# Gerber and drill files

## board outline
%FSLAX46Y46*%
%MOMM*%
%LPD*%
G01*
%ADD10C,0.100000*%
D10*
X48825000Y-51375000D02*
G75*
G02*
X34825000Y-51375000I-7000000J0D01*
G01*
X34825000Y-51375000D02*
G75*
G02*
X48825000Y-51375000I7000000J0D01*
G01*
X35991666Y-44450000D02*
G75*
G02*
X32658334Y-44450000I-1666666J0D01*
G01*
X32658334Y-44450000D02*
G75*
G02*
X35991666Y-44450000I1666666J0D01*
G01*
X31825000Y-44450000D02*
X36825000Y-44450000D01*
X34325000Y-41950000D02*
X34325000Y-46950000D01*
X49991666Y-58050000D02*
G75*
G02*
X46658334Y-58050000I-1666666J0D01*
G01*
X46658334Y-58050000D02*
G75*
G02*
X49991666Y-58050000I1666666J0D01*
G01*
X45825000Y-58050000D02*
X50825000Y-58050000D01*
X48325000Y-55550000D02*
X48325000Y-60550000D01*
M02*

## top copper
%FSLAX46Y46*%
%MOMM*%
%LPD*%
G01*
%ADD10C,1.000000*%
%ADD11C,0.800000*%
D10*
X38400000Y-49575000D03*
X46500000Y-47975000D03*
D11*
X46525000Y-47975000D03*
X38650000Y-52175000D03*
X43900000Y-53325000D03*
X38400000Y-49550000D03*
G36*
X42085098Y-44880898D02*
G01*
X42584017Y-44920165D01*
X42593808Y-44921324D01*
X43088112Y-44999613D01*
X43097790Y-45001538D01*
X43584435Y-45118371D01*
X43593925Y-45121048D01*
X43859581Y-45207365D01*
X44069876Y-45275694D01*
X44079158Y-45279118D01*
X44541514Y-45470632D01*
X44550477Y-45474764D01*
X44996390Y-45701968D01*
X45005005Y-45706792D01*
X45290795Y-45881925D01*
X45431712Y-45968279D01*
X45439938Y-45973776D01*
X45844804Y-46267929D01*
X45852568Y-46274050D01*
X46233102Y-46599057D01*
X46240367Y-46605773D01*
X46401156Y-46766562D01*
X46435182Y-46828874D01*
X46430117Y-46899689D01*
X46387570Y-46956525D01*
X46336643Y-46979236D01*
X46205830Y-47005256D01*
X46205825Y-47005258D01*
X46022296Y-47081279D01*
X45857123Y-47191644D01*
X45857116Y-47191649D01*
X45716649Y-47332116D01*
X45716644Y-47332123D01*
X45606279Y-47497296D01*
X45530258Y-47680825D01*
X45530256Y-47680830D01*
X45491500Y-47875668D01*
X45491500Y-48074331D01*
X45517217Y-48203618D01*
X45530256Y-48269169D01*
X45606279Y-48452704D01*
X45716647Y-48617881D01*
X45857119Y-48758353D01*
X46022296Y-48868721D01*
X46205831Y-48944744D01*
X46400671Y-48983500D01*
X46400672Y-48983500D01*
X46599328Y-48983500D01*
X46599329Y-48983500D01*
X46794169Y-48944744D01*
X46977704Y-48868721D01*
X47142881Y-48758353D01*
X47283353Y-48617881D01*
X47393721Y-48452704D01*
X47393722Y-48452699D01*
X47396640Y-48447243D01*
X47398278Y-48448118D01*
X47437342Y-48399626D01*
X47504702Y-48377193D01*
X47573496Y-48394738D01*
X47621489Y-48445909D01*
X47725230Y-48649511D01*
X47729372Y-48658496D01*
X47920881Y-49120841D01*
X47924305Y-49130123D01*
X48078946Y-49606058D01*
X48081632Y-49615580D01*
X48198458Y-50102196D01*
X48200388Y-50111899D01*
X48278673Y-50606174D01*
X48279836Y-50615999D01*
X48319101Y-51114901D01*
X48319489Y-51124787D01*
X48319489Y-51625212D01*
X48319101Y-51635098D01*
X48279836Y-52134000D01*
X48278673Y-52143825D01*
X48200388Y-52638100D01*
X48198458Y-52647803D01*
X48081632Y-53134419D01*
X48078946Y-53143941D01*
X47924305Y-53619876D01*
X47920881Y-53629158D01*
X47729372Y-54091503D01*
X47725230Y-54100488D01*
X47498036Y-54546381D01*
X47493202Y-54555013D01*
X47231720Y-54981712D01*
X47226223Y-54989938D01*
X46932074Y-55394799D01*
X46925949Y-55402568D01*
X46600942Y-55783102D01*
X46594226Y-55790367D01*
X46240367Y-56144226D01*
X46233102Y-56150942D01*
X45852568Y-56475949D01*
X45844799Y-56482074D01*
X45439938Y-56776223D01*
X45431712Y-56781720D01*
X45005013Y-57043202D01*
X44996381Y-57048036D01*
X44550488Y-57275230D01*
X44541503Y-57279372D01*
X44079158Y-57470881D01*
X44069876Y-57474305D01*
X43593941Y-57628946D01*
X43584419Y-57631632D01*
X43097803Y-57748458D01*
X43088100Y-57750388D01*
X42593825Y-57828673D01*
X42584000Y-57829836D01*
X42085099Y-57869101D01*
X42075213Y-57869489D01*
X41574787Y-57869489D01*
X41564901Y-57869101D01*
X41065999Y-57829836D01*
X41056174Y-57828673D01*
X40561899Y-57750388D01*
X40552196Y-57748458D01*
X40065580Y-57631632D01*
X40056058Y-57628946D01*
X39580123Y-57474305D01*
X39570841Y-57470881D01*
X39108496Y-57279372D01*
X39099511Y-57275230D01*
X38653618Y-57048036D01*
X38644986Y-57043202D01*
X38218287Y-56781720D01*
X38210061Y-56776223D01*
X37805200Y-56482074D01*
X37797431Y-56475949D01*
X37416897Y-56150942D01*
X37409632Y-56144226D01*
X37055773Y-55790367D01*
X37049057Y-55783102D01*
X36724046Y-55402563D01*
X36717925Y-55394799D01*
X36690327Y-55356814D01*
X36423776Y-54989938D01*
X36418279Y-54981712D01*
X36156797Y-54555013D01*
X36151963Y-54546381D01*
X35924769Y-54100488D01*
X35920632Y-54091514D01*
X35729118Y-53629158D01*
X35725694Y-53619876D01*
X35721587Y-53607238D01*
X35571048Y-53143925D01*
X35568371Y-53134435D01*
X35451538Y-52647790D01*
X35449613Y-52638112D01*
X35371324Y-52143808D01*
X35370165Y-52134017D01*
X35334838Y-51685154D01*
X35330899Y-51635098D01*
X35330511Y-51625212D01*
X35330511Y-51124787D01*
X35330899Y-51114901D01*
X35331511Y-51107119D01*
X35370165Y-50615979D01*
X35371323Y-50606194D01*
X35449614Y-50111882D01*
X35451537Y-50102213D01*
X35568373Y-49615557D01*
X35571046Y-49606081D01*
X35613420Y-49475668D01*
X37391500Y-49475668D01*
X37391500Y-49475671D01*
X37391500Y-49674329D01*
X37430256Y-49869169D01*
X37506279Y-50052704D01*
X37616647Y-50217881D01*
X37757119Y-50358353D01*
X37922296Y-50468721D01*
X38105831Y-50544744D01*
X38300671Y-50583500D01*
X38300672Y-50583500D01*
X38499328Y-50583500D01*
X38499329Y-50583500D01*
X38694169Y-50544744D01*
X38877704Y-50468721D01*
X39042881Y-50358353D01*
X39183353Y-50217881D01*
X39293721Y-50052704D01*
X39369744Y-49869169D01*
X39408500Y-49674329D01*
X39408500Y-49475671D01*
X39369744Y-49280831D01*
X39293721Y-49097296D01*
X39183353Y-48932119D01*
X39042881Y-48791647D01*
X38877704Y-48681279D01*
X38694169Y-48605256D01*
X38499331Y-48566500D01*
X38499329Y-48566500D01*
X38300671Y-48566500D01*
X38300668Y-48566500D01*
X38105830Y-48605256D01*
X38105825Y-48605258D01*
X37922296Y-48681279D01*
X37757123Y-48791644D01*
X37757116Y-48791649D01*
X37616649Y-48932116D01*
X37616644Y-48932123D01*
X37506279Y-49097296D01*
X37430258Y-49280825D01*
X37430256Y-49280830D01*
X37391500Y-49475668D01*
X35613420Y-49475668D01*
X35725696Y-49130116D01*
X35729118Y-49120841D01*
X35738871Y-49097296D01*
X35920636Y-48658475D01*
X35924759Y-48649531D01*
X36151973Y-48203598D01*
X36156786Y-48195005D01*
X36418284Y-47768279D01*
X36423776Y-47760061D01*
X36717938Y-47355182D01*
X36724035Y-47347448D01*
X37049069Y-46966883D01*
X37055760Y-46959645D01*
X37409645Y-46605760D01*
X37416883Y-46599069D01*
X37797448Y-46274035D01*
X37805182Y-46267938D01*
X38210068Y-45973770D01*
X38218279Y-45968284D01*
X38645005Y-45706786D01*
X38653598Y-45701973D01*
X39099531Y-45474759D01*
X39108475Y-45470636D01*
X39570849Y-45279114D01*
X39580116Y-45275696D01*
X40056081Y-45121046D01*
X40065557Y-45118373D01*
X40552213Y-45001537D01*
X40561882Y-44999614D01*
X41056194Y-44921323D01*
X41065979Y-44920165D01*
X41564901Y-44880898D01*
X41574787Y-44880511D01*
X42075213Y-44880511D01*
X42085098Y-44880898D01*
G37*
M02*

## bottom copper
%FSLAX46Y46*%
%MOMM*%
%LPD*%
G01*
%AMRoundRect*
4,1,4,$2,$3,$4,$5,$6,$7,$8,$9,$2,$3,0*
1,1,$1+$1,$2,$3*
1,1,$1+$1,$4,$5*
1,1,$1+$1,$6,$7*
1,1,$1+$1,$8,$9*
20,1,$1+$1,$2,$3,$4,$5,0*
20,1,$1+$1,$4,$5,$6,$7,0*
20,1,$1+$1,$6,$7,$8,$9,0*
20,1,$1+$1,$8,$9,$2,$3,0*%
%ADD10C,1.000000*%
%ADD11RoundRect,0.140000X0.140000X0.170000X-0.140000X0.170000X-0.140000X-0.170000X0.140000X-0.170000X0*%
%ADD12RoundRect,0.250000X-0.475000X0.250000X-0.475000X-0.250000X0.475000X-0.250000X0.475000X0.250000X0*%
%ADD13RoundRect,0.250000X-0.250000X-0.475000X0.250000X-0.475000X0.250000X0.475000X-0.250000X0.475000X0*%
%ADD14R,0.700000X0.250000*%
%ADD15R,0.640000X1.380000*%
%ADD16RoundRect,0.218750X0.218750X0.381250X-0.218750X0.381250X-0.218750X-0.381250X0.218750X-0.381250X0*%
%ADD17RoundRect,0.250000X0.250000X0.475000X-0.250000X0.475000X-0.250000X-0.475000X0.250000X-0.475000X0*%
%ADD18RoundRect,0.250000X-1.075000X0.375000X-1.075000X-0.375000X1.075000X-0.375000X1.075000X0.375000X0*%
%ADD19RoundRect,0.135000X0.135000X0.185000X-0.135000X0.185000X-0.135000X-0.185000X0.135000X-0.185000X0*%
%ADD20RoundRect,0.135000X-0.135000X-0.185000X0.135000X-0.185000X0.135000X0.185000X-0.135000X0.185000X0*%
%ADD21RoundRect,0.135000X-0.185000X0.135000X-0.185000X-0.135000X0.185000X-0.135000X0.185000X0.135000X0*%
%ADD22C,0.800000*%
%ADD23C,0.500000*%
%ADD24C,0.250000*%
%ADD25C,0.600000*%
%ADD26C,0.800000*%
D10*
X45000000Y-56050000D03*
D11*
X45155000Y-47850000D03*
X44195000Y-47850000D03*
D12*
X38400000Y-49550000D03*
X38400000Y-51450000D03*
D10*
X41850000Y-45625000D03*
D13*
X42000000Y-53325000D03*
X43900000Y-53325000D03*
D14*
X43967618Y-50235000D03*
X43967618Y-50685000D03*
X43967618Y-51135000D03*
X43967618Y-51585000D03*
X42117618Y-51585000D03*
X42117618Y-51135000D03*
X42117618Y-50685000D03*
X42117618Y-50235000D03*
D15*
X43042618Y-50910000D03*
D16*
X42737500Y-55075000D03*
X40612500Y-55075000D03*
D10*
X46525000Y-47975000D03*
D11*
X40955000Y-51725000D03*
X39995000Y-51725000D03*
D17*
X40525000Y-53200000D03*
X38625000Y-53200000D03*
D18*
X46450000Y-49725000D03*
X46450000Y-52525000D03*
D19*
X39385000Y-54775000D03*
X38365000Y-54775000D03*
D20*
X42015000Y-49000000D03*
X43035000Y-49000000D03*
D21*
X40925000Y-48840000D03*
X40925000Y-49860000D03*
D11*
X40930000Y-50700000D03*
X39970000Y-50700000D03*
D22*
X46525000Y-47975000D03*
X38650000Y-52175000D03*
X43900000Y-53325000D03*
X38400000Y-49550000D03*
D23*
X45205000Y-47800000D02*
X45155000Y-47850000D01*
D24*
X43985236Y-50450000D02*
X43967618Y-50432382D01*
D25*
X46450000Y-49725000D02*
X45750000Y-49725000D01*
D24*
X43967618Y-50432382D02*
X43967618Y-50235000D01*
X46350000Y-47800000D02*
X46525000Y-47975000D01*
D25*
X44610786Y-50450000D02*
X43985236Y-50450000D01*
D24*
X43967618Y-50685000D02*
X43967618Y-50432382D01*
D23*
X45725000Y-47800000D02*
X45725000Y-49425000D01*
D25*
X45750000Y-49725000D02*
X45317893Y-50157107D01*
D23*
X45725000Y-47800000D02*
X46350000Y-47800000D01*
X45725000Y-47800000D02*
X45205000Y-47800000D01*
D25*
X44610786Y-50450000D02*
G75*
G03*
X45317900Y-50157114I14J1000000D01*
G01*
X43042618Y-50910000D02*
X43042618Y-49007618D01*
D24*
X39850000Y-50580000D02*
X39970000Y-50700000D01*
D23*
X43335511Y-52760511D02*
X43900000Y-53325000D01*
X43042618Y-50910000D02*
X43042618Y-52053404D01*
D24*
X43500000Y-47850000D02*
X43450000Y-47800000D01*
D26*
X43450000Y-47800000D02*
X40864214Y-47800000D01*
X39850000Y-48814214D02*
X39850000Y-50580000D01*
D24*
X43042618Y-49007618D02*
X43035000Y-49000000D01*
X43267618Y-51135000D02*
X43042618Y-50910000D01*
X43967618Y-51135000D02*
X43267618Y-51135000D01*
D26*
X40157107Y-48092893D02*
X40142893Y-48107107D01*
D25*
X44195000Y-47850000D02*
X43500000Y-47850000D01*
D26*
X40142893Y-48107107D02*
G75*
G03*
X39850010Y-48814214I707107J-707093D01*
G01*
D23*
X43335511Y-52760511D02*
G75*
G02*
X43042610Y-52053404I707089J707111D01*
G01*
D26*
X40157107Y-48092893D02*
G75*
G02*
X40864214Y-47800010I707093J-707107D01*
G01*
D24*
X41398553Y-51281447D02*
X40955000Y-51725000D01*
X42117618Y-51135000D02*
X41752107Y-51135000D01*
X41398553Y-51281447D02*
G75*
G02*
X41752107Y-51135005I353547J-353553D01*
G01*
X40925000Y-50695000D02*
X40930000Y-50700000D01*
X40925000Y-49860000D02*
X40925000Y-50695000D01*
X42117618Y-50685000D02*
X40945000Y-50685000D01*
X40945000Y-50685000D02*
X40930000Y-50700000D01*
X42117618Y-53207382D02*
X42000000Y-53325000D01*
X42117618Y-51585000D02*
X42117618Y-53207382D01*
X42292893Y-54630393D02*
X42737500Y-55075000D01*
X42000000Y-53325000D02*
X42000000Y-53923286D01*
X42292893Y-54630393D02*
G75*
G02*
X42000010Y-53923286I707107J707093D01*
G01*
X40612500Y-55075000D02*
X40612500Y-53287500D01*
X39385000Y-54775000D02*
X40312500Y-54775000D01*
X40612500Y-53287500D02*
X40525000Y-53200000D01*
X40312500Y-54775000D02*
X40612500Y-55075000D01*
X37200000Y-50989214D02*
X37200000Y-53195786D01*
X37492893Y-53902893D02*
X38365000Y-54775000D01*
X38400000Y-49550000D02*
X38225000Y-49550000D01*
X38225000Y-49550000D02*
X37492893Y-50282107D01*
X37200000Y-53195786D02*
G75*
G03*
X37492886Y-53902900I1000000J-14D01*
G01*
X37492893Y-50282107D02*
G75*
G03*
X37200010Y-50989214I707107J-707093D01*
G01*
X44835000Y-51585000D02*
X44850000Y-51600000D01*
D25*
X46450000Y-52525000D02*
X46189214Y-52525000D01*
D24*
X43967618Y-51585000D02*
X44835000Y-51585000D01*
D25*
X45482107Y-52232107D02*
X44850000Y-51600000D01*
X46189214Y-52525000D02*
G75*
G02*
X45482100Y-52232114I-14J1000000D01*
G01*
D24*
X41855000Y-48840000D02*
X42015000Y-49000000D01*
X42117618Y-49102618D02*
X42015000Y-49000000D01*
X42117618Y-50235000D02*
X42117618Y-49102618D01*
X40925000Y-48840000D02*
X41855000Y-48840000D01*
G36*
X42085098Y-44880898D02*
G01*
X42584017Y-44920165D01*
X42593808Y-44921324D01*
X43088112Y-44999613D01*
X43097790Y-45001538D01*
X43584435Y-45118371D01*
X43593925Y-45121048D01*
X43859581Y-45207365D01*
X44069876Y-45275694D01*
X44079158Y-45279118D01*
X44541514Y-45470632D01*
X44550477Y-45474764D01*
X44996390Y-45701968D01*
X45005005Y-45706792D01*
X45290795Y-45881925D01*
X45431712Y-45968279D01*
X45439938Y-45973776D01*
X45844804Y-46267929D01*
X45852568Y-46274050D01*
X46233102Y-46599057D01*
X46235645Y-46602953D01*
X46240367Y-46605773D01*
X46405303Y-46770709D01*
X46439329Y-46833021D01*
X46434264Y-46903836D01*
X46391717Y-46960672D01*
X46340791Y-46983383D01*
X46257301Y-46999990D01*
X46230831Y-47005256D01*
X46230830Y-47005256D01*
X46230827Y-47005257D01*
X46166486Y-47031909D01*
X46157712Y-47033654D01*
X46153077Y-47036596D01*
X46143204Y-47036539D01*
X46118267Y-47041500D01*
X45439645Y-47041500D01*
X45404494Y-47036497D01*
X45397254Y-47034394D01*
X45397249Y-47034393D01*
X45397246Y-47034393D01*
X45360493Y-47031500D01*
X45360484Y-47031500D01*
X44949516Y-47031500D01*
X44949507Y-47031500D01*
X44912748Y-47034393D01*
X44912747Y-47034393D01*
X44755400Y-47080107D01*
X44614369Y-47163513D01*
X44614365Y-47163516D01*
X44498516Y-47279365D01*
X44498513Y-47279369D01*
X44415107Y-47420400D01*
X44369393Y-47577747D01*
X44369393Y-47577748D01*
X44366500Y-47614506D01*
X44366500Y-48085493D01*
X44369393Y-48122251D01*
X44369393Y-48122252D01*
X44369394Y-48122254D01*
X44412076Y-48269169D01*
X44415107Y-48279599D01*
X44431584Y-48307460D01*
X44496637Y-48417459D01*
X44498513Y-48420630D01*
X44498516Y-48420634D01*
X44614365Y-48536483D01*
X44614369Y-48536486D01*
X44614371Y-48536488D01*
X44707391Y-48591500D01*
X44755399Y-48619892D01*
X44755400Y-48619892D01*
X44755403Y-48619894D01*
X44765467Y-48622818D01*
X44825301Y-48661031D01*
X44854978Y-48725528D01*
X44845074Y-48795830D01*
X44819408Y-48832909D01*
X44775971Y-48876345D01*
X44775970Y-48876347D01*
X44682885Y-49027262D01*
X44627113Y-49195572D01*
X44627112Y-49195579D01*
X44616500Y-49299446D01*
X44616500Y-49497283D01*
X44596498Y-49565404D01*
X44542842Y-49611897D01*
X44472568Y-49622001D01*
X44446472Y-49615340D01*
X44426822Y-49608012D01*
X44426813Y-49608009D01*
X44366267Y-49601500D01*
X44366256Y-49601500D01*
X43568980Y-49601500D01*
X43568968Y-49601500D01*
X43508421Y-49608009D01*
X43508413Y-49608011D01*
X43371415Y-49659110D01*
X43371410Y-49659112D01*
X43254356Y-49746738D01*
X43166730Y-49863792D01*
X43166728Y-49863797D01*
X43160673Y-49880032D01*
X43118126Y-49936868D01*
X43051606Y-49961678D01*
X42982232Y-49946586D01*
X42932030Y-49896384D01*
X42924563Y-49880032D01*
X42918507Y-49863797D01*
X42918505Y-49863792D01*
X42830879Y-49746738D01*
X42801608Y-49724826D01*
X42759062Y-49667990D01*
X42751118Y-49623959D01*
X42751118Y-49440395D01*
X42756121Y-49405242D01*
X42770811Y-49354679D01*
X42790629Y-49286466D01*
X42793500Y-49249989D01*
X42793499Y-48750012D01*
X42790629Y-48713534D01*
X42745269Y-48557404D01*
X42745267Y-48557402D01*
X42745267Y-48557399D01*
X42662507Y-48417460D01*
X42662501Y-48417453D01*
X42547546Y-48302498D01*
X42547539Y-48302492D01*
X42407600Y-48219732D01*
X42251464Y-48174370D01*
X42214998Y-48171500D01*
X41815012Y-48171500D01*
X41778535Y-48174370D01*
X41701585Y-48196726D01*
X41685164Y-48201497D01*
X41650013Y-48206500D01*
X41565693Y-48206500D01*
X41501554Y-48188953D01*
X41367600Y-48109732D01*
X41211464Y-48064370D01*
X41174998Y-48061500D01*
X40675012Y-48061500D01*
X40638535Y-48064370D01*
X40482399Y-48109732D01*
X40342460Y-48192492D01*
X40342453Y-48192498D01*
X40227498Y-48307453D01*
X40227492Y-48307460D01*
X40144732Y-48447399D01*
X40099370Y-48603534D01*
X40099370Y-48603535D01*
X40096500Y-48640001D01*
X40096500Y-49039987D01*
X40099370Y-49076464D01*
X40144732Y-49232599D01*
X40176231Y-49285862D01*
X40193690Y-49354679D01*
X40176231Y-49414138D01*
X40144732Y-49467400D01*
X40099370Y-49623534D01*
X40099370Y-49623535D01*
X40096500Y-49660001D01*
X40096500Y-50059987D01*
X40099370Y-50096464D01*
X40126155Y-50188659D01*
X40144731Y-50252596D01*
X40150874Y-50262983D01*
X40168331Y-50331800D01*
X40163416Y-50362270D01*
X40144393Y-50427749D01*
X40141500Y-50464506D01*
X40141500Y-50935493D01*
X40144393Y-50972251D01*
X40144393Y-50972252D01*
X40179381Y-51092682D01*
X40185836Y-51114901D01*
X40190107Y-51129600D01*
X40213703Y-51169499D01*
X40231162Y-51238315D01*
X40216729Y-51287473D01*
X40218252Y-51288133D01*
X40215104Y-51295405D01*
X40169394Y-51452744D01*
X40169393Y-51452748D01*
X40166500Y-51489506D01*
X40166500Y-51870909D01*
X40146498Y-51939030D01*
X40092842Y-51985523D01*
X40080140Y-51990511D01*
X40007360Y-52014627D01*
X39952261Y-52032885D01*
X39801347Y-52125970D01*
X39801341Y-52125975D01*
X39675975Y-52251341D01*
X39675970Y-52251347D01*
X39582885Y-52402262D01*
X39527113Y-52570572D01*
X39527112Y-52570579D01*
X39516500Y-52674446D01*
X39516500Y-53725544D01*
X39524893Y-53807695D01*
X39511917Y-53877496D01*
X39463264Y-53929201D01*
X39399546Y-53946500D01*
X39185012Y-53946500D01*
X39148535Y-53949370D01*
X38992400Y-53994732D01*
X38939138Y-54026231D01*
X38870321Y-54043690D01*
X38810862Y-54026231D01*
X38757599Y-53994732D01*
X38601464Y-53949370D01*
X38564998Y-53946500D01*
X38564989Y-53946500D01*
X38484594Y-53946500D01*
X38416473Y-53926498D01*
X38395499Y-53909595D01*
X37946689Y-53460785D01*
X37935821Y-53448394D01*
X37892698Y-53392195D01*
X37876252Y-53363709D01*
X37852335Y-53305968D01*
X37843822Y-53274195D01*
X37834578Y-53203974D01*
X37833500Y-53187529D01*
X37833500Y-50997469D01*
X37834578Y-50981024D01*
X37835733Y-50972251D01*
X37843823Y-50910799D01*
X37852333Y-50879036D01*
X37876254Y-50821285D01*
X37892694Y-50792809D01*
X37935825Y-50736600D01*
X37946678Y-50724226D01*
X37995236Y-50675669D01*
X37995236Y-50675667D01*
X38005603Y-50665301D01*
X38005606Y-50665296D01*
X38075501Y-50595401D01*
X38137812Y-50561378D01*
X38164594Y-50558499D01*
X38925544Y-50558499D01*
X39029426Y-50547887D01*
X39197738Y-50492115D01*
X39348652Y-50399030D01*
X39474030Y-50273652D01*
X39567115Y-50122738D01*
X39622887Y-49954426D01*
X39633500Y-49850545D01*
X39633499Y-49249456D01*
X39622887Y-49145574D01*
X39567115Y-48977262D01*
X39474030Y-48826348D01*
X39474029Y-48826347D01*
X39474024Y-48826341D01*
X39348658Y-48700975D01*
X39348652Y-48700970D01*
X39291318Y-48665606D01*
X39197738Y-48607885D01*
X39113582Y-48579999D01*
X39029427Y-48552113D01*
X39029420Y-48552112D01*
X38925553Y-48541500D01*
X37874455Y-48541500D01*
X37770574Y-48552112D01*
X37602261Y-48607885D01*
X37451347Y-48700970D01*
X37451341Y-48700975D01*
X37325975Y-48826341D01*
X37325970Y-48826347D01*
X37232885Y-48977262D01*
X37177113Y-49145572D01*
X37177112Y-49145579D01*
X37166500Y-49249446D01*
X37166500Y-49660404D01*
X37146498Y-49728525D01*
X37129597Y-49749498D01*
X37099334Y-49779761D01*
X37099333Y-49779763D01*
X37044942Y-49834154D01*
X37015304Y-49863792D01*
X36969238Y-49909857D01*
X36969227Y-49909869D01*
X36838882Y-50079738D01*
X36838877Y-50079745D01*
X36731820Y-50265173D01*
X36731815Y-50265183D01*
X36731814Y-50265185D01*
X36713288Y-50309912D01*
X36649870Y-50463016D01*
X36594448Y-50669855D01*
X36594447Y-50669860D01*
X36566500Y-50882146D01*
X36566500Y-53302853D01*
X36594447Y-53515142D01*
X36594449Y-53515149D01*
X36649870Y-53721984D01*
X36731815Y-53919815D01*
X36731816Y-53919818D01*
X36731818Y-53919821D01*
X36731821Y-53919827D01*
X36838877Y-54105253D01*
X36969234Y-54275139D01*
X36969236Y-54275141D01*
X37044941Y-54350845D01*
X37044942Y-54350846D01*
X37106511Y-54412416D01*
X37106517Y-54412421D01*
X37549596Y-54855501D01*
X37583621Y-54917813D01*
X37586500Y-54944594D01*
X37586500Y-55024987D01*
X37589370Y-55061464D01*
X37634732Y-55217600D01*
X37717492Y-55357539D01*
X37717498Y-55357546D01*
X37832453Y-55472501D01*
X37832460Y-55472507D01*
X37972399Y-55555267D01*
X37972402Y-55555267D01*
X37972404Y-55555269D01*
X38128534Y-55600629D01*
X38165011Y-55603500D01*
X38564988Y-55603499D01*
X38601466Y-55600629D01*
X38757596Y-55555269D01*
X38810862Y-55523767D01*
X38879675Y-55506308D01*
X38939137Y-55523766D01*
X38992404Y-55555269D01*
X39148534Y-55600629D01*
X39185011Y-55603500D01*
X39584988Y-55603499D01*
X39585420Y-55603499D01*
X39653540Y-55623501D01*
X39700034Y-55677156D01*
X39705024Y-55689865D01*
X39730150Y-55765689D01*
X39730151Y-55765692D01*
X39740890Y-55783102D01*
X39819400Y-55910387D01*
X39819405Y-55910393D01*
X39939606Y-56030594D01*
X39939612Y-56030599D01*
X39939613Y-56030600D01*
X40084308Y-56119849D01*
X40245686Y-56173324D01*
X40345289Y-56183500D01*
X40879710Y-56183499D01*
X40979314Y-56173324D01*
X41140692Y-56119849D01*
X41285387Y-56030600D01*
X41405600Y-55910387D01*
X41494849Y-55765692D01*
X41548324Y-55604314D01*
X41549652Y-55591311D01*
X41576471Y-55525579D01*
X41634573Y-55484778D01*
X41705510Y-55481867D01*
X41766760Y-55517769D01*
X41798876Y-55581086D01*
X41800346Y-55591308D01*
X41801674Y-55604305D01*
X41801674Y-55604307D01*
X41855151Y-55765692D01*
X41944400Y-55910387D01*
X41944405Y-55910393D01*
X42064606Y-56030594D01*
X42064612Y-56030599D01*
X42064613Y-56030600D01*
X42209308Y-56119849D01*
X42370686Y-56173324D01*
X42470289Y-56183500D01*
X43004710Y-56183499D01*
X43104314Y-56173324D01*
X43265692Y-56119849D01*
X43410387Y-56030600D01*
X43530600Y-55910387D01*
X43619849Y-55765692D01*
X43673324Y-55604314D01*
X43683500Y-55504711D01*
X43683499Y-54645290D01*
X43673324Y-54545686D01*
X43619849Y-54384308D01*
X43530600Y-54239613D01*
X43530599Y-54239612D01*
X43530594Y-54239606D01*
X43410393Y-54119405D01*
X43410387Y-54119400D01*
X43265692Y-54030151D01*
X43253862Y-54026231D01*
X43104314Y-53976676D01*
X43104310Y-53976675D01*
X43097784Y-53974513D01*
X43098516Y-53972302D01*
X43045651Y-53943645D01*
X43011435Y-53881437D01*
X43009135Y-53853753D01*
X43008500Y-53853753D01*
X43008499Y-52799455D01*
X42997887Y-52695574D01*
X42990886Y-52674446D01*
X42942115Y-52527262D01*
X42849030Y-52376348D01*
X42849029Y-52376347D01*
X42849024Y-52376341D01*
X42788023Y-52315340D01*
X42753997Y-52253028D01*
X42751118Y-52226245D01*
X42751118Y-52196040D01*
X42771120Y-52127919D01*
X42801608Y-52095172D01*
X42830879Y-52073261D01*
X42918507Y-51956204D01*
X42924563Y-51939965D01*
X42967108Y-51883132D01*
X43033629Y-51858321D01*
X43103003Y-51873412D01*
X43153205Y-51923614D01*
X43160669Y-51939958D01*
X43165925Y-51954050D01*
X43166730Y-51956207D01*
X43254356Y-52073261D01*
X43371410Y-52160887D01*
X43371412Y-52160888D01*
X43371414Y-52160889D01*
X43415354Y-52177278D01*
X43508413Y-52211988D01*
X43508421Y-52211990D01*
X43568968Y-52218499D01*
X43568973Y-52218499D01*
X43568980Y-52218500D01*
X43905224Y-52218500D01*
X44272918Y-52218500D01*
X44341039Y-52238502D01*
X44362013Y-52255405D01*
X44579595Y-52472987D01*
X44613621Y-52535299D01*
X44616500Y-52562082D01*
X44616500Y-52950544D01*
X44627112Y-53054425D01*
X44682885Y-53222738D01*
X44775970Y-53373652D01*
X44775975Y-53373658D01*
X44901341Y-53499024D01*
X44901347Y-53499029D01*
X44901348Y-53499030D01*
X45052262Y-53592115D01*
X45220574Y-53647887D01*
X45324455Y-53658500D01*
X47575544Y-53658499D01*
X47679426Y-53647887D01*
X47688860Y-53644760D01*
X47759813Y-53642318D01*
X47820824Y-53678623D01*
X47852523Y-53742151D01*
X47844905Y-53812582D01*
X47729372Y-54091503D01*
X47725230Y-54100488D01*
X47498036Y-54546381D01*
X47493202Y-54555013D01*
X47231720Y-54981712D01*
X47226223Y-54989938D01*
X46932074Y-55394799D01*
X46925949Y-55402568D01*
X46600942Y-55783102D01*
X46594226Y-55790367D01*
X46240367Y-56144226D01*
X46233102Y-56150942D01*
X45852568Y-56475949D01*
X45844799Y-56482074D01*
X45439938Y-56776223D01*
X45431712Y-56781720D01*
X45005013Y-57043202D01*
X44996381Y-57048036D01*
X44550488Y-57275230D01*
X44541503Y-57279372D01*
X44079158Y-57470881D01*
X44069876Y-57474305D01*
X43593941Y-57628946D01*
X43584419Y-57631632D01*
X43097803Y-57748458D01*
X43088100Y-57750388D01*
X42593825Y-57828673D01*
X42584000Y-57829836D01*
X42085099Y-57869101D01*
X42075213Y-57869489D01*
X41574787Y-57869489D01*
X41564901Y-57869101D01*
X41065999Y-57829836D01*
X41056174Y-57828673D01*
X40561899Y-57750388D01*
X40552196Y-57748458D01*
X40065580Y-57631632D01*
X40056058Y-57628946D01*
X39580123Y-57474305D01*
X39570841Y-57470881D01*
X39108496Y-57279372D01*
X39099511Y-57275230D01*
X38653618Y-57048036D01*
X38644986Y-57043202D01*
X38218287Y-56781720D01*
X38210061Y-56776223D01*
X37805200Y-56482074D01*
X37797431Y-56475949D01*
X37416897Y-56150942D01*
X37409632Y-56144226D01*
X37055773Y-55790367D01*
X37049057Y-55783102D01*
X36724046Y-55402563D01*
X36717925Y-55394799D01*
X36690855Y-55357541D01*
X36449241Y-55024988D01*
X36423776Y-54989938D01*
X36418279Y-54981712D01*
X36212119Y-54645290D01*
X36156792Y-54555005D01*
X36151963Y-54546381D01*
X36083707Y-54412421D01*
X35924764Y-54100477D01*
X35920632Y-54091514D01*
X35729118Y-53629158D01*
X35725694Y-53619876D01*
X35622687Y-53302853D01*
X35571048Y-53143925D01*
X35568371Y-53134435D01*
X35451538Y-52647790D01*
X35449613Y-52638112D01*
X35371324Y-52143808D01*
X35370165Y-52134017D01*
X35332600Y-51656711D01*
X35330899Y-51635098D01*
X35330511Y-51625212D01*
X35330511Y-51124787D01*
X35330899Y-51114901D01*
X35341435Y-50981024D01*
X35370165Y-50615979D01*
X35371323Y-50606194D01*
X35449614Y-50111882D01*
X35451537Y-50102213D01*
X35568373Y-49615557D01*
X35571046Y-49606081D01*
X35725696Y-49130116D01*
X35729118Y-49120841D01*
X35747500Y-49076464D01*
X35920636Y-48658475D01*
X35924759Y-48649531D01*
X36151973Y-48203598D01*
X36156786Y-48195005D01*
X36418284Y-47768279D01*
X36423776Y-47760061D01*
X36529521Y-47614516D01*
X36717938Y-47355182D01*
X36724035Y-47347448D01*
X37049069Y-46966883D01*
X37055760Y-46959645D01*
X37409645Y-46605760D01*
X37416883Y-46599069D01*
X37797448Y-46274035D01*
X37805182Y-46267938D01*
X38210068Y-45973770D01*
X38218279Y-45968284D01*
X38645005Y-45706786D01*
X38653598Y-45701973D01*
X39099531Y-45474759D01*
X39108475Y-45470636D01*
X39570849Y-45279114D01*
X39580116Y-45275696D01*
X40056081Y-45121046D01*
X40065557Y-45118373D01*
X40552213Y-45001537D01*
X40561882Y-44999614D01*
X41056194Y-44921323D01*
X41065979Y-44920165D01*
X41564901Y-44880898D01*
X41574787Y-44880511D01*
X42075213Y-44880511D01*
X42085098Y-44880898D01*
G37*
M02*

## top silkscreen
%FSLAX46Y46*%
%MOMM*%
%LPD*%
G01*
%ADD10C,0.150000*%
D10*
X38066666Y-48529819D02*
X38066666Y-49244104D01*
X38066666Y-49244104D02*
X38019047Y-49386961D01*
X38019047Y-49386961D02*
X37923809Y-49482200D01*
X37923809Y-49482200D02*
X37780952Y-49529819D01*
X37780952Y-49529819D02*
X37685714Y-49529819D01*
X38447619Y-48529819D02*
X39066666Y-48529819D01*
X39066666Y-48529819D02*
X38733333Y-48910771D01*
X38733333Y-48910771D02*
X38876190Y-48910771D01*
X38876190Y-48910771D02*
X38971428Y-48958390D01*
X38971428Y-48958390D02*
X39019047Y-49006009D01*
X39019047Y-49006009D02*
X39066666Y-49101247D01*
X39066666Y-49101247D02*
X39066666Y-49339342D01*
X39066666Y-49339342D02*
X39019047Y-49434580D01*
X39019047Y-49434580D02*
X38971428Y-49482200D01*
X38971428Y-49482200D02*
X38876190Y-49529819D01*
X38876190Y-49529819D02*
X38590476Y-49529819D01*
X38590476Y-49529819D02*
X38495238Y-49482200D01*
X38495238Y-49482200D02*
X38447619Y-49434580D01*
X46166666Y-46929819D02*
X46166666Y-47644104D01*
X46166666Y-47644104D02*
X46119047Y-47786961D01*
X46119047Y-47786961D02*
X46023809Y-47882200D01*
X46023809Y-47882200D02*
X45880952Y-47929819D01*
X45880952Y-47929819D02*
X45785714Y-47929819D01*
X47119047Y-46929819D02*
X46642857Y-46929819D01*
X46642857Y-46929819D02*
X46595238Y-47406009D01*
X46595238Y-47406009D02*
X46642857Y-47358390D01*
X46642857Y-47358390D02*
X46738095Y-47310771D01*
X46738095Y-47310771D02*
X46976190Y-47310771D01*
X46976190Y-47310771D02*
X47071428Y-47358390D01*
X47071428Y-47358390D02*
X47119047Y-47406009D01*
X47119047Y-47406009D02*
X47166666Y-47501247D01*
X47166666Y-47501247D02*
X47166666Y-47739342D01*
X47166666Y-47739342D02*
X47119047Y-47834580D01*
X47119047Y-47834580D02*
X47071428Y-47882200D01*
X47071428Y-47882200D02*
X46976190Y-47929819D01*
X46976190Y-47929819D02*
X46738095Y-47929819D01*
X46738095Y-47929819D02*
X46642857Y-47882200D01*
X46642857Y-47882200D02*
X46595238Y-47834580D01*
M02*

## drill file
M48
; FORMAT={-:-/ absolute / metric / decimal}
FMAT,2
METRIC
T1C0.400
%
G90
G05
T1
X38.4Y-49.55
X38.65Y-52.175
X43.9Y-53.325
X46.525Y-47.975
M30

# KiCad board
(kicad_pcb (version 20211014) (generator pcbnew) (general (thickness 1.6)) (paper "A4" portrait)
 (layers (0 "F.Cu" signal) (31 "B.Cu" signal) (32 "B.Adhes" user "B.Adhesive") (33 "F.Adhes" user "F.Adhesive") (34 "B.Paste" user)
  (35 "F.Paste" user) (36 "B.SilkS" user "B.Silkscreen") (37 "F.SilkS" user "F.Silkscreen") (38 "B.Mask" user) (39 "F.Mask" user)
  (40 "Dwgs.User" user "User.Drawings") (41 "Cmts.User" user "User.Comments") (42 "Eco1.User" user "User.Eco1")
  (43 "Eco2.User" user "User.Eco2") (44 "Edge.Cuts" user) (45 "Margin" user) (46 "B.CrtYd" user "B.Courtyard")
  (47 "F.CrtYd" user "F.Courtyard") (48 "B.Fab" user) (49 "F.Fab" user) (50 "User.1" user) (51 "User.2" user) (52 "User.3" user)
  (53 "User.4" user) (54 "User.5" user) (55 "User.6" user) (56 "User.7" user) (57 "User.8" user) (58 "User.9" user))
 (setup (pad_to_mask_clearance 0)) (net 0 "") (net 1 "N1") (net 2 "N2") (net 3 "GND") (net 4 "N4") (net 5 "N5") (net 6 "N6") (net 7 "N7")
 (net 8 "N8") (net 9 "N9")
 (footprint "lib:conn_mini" (layer "F.Cu") (at 38.4 49.575)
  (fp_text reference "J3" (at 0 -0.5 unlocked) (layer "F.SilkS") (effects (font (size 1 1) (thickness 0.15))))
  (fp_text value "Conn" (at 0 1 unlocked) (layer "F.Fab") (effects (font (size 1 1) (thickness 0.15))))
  (pad "1" smd circle (at 0 0) (size 1 1) (layers "F.Cu" "F.Paste" "F.Mask") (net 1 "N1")))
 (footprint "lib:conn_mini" (layer "F.Cu") (at 46.5 47.975)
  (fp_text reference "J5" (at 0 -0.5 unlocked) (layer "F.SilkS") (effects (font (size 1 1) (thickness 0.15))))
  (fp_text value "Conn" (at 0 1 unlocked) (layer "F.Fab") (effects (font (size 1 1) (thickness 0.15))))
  (pad "1" smd circle (at 0 0) (size 1 1) (layers "F.Cu" "F.Paste" "F.Mask") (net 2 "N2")))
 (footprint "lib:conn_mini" (layer "B.Cu") (at 45 56.05 180)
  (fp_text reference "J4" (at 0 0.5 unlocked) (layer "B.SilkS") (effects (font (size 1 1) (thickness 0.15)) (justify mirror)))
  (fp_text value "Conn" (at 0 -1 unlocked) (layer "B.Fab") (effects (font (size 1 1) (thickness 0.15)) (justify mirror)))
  (pad "1" smd circle (at 0 0 180) (size 1 1) (layers "B.Cu" "B.Paste" "B.Mask") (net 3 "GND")))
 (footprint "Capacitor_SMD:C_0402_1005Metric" (layer "B.Cu") (at 44.675 47.85 180)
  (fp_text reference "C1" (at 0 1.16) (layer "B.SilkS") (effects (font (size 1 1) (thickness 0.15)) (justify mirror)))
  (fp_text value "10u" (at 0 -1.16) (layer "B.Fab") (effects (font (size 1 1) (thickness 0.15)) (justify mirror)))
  (pad "1" smd roundrect (at -0.48 0 180) (size 0.56 0.62) (layers "B.Cu" "B.Paste" "B.Mask") (roundrect_rratio 0.25) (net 2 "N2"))
  (pad "2" smd roundrect (at 0.48 0 180) (size 0.56 0.62) (layers "B.Cu" "B.Paste" "B.Mask") (roundrect_rratio 0.25) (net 3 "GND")))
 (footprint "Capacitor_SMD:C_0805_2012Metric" (layer "B.Cu") (at 38.4 50.5 -90)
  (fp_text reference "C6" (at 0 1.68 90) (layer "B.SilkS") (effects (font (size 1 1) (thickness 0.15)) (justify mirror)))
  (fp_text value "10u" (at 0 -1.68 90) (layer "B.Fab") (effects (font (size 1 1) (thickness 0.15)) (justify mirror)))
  (pad "1" smd roundrect (at -0.95 0 270) (size 1 1.45) (layers "B.Cu" "B.Paste" "B.Mask") (roundrect_rratio 0.25) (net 1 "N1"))
  (pad "2" smd roundrect (at 0.95 0 270) (size 1 1.45) (layers "B.Cu" "B.Paste" "B.Mask") (roundrect_rratio 0.25) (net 3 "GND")))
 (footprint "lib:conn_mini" (layer "B.Cu") (at 41.85 45.625 180)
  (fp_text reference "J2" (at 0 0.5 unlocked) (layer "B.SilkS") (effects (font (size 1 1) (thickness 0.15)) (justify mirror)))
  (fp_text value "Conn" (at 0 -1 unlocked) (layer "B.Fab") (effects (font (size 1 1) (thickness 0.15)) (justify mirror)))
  (pad "1" smd circle (at 0 0 180) (size 1 1) (layers "B.Cu" "B.Paste" "B.Mask") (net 3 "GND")))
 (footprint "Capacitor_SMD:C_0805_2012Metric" (layer "B.Cu") (at 42.95 53.325)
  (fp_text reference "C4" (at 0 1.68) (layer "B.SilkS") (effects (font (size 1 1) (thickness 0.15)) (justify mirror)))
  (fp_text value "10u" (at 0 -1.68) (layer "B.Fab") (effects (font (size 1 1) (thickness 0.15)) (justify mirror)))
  (pad "1" smd roundrect (at -0.95 0) (size 1 1.45) (layers "B.Cu" "B.Paste" "B.Mask") (roundrect_rratio 0.25) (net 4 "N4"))
  (pad "2" smd roundrect (at 0.95 0) (size 1 1.45) (layers "B.Cu" "B.Paste" "B.Mask") (roundrect_rratio 0.25) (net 3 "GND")))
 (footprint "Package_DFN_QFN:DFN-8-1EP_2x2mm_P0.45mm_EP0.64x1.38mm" (layer "B.Cu") (at 43.042618 50.91 180)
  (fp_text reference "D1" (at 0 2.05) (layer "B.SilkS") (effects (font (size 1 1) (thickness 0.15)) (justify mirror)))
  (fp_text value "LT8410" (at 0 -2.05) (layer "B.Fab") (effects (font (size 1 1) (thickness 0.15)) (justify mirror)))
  (pad "" smd rect (at 0 -0.345 180) (size 0.53 0.54) (layers "B.Paste"))
  (pad "" smd rect (at 0 0.345 180) (size 0.53 0.54) (layers "B.Paste"))
  (pad "1" smd rect (at -0.925 0.675 180) (size 0.7 0.25) (layers "B.Cu" "B.Paste" "B.Mask") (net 2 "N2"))
  (pad "2" smd rect (at -0.925 0.225 180) (size 0.7 0.25) (layers "B.Cu" "B.Paste" "B.Mask") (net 2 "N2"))
  (pad "3" smd rect (at -0.925 -0.225 180) (size 0.7 0.25) (layers "B.Cu" "B.Paste" "B.Mask") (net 3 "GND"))
  (pad "4" smd rect (at -0.925 -0.675 180) (size 0.7 0.25) (layers "B.Cu" "B.Paste" "B.Mask") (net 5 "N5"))
  (pad "5" smd rect (at 0.925 -0.675 180) (size 0.7 0.25) (layers "B.Cu" "B.Paste" "B.Mask") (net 4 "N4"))
  (pad "6" smd rect (at 0.925 -0.225 180) (size 0.7 0.25) (layers "B.Cu" "B.Paste" "B.Mask") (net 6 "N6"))
  (pad "7" smd rect (at 0.925 0.225 180) (size 0.7 0.25) (layers "B.Cu" "B.Paste" "B.Mask") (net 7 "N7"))
  (pad "8" smd rect (at 0.925 0.675 180) (size 0.7 0.25) (layers "B.Cu" "B.Paste" "B.Mask") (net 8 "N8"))
  (pad "9" smd rect (at 0 0 180) (size 0.64 1.38) (layers "B.Cu" "B.Mask") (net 3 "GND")))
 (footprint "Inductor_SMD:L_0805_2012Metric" (layer "B.Cu") (at 41.675 55.075 180)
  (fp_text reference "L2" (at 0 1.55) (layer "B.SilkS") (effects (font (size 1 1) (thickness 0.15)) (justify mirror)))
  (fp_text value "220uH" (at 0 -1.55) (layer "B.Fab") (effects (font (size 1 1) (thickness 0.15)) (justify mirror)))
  (pad "1" smd roundrect (at -1.0625 0 180) (size 0.875 1.2) (layers "B.Cu" "B.Paste" "B.Mask") (roundrect_rratio 0.25) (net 4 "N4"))
  (pad "2" smd roundrect (at 1.0625 0 180) (size 0.875 1.2) (layers "B.Cu" "B.Paste" "B.Mask") (roundrect_rratio 0.25) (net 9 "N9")))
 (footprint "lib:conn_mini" (layer "B.Cu") (at 46.525 47.975 180)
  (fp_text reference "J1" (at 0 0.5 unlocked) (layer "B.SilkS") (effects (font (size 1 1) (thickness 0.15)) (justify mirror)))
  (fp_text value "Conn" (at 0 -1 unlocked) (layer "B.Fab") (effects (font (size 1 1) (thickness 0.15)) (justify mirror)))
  (pad "1" smd circle (at 0 0 180) (size 1 1) (layers "B.Cu" "B.Paste" "B.Mask") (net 2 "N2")))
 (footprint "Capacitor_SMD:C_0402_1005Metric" (layer "B.Cu") (at 40.475 51.725 180)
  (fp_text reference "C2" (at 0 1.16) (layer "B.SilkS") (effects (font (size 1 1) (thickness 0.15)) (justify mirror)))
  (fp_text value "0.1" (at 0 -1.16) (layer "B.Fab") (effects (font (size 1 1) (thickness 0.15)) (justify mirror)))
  (pad "1" smd roundrect (at -0.48 0 180) (size 0.56 0.62) (layers "B.Cu" "B.Paste" "B.Mask") (roundrect_rratio 0.25) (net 6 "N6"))
  (pad "2" smd roundrect (at 0.48 0 180) (size 0.56 0.62) (layers "B.Cu" "B.Paste" "B.Mask") (roundrect_rratio 0.25) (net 3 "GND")))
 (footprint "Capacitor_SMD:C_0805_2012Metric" (layer "B.Cu") (at 39.575 53.2 180)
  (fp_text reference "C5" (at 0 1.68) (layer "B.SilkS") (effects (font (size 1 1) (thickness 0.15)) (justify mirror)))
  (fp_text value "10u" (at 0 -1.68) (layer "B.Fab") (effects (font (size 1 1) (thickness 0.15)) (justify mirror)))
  (pad "1" smd roundrect (at -0.95 0 180) (size 1 1.45) (layers "B.Cu" "B.Paste" "B.Mask") (roundrect_rratio 0.25) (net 9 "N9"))
  (pad "2" smd roundrect (at 0.95 0 180) (size 1 1.45) (layers "B.Cu" "B.Paste" "B.Mask") (roundrect_rratio 0.25) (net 3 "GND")))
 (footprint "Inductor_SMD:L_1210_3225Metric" (layer "B.Cu") (at 46.45 51.125 -90)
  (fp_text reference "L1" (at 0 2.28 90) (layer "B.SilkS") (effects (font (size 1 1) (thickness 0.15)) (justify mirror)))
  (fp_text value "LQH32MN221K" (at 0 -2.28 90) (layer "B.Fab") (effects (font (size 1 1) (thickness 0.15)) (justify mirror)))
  (pad "1" smd roundrect (at -1.4 0 270) (size 1.25 2.65) (layers "B.Cu" "B.Paste" "B.Mask") (roundrect_rratio 0.2) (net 2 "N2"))
  (pad "2" smd roundrect (at 1.4 0 270) (size 1.25 2.65) (layers "B.Cu" "B.Paste" "B.Mask") (roundrect_rratio 0.2) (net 5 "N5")))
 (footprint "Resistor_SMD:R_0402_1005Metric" (layer "B.Cu") (at 38.875 54.775 180)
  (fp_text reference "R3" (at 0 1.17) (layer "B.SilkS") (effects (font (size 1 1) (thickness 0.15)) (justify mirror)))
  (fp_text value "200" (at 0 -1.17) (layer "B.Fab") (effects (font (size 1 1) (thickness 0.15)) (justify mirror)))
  (pad "1" smd roundrect (at -0.51 0 180) (size 0.54 0.64) (layers "B.Cu" "B.Paste" "B.Mask") (roundrect_rratio 0.25) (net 9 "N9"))
  (pad "2" smd roundrect (at 0.51 0 180) (size 0.54 0.64) (layers "B.Cu" "B.Paste" "B.Mask") (roundrect_rratio 0.25) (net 1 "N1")))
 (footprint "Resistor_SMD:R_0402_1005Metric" (layer "B.Cu") (at 42.525 49)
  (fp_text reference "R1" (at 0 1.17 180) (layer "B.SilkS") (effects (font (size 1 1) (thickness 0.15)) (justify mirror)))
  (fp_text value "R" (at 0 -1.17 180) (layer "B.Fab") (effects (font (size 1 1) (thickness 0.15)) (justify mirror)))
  (pad "1" smd roundrect (at -0.51 0) (size 0.54 0.64) (layers "B.Cu" "B.Paste" "B.Mask") (roundrect_rratio 0.25) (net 8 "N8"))
  (pad "2" smd roundrect (at 0.51 0) (size 0.54 0.64) (layers "B.Cu" "B.Paste" "B.Mask") (roundrect_rratio 0.25) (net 3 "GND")))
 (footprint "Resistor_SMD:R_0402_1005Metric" (layer "B.Cu") (at 40.925 49.35 -90)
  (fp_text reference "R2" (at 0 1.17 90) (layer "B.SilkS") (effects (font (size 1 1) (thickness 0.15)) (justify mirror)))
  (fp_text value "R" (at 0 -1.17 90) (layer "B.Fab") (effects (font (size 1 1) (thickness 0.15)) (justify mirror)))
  (pad "1" smd roundrect (at -0.51 0 270) (size 0.54 0.64) (layers "B.Cu" "B.Paste" "B.Mask") (roundrect_rratio 0.25) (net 8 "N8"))
  (pad "2" smd roundrect (at 0.51 0 270) (size 0.54 0.64) (layers "B.Cu" "B.Paste" "B.Mask") (roundrect_rratio 0.25) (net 7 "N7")))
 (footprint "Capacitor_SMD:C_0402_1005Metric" (layer "B.Cu") (at 40.45 50.7 180)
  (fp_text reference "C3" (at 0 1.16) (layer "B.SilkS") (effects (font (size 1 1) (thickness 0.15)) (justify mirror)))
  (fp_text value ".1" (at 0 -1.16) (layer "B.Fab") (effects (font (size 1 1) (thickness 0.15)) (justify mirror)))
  (pad "1" smd roundrect (at -0.48 0 180) (size 0.56 0.62) (layers "B.Cu" "B.Paste" "B.Mask") (roundrect_rratio 0.25) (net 7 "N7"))
  (pad "2" smd roundrect (at 0.48 0 180) (size 0.56 0.62) (layers "B.Cu" "B.Paste" "B.Mask") (roundrect_rratio 0.25) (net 3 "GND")))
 (gr_circle (center 41.825 51.375) (end 48.825 51.375) (layer "Edge.Cuts") (width 0.1) (fill none))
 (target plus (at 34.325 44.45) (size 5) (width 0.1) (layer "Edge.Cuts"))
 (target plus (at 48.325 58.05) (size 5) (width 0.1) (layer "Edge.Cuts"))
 (via (at 46.525 47.975) (size 0.8) (drill 0.4) (layers "F.Cu" "B.Cu") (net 2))
 (segment (start 45.205 47.8) (end 45.155 47.85) (width 0.5) (layer "B.Cu") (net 2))
 (segment (start 43.985236 50.45) (end 43.967618 50.432382) (width 0.25) (layer "B.Cu") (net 2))
 (segment (start 46.45 49.725) (end 45.75 49.725) (width 0.6) (layer "B.Cu") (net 2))
 (segment (start 43.967618 50.432382) (end 43.967618 50.235) (width 0.25) (layer "B.Cu") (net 2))
 (segment (start 46.35 47.8) (end 46.525 47.975) (width 0.25) (layer "B.Cu") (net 2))
 (segment (start 44.610786 50.45) (end 43.985236 50.45) (width 0.6) (layer "B.Cu") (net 2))
 (segment (start 43.967618 50.685) (end 43.967618 50.432382) (width 0.25) (layer "B.Cu") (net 2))
 (segment (start 45.725 47.8) (end 45.725 49.425) (width 0.5) (layer "B.Cu") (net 2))
 (segment (start 45.75 49.725) (end 45.317893 50.157107) (width 0.6) (layer "B.Cu") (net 2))
 (segment (start 45.725 47.8) (end 46.35 47.8) (width 0.5) (layer "B.Cu") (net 2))
 (segment (start 45.725 47.8) (end 45.205 47.8) (width 0.5) (layer "B.Cu") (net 2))
 (arc (start 44.610786 50.45) (mid 44.993469 50.37388) (end 45.317893 50.157107) (width 0.6) (layer "B.Cu") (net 2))
 (via (at 38.65 52.175) (size 0.8) (drill 0.4) (layers "F.Cu" "B.Cu") (free) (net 3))
 (via (at 43.9 53.325) (size 0.8) (drill 0.4) (layers "F.Cu" "B.Cu") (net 3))
 (segment (start 43.042618 50.91) (end 43.042618 49.007618) (width 0.6) (layer "B.Cu") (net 3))
 (segment (start 39.85 50.58) (end 39.97 50.7) (width 0.25) (layer "B.Cu") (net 3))
 (segment (start 43.335511 52.760511) (end 43.9 53.325) (width 0.5) (layer "B.Cu") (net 3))
 (segment (start 43.042618 50.91) (end 43.042618 52.053404) (width 0.5) (layer "B.Cu") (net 3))
 (segment (start 43.5 47.85) (end 43.45 47.8) (width 0.25) (layer "B.Cu") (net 3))
 (segment (start 43.45 47.8) (end 40.864214 47.8) (width 0.8) (layer "B.Cu") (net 3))
 (segment (start 39.85 48.814214) (end 39.85 50.58) (width 0.8) (layer "B.Cu") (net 3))
 (segment (start 43.042618 49.007618) (end 43.035 49) (width 0.25) (layer "B.Cu") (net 3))
 (segment (start 43.267618 51.135) (end 43.042618 50.91) (width 0.25) (layer "B.Cu") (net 3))
 (segment (start 43.967618 51.135) (end 43.267618 51.135) (width 0.25) (layer "B.Cu") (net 3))
 (segment (start 40.157107 48.092893) (end 40.142893 48.107107) (width 0.8) (layer "B.Cu") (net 3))
 (segment (start 44.195 47.85) (end 43.5 47.85) (width 0.6) (layer "B.Cu") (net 3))
 (arc (start 40.142893 48.107107) (mid 39.92612 48.43153) (end 39.85 48.814214) (width 0.8) (layer "B.Cu") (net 3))
 (arc (start 43.335511 52.760511) (mid 43.118738 52.436088) (end 43.042618 52.053404) (width 0.5) (layer "B.Cu") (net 3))
 (arc (start 40.157107 48.092893) (mid 40.48153 47.87612) (end 40.864214 47.8) (width 0.8) (layer "B.Cu") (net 3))
 (segment (start 41.398553 51.281447) (end 40.955 51.725) (width 0.25) (layer "B.Cu") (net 6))
 (segment (start 42.117618 51.135) (end 41.752107 51.135) (width 0.25) (layer "B.Cu") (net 6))
 (arc (start 41.398553 51.281447) (mid 41.560765 51.17306) (end 41.752107 51.135) (width 0.25) (layer "B.Cu") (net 6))
 (segment (start 40.925 50.695) (end 40.93 50.7) (width 0.25) (layer "B.Cu") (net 7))
 (segment (start 40.925 49.86) (end 40.925 50.695) (width 0.25) (layer "B.Cu") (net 7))
 (segment (start 42.117618 50.685) (end 40.945 50.685) (width 0.25) (layer "B.Cu") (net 7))
 (segment (start 40.945 50.685) (end 40.93 50.7) (width 0.25) (layer "B.Cu") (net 7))
 (segment (start 42.117618 53.207382) (end 42 53.325) (width 0.25) (layer "B.Cu") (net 4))
 (segment (start 42.117618 51.585) (end 42.117618 53.207382) (width 0.25) (layer "B.Cu") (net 4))
 (segment (start 42.292893 54.630393) (end 42.7375 55.075) (width 0.25) (layer "B.Cu") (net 4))
 (segment (start 42 53.325) (end 42 53.923286) (width 0.25) (layer "B.Cu") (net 4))
 (arc (start 42.292893 54.630393) (mid 42.07612 54.30597) (end 42 53.923286) (width 0.25) (layer "B.Cu") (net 4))
 (segment (start 40.6125 55.075) (end 40.6125 53.2875) (width 0.25) (layer "B.Cu") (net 9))
 (segment (start 39.385 54.775) (end 40.3125 54.775) (width 0.25) (layer "B.Cu") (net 9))
 (segment (start 40.6125 53.2875) (end 40.525 53.2) (width 0.25) (layer "B.Cu") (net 9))
 (segment (start 40.3125 54.775) (end 40.6125 55.075) (width 0.25) (layer "B.Cu") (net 9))
 (via (at 38.4 49.55) (size 0.8) (drill 0.4) (layers "F.Cu" "B.Cu") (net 1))
 (segment (start 37.2 50.989214) (end 37.2 53.195786) (width 0.25) (layer "B.Cu") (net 1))
 (segment (start 37.492893 53.902893) (end 38.365 54.775) (width 0.25) (layer "B.Cu") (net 1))
 (segment (start 38.4 49.55) (end 38.225 49.55) (width 0.25) (layer "B.Cu") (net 1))
 (segment (start 38.225 49.55) (end 37.492893 50.282107) (width 0.25) (layer "B.Cu") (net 1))
 (arc (start 37.2 53.195786) (mid 37.27612 53.578469) (end 37.492893 53.902893) (width 0.25) (layer "B.Cu") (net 1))
 (arc (start 37.492893 50.282107) (mid 37.27612 50.60653) (end 37.2 50.989214) (width 0.25) (layer "B.Cu") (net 1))
 (segment (start 44.835 51.585) (end 44.85 51.6) (width 0.25) (layer "B.Cu") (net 5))
 (segment (start 46.45 52.525) (end 46.189214 52.525) (width 0.6) (layer "B.Cu") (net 5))
 (segment (start 43.967618 51.585) (end 44.835 51.585) (width 0.25) (layer "B.Cu") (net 5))
 (segment (start 45.482107 52.232107) (end 44.85 51.6) (width 0.6) (layer "B.Cu") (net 5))
 (arc (start 46.189214 52.525) (mid 45.806531 52.44888) (end 45.482107 52.232107) (width 0.6) (layer "B.Cu") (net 5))
 (segment (start 41.855 48.84) (end 42.015 49) (width 0.25) (layer "B.Cu") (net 8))
 (segment (start 42.117618 49.102618) (end 42.015 49) (width 0.25) (layer "B.Cu") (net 8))
 (segment (start 42.117618 50.235) (end 42.117618 49.102618) (width 0.25) (layer "B.Cu") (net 8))
 (segment (start 40.925 48.84) (end 41.855 48.84) (width 0.25) (layer "B.Cu") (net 8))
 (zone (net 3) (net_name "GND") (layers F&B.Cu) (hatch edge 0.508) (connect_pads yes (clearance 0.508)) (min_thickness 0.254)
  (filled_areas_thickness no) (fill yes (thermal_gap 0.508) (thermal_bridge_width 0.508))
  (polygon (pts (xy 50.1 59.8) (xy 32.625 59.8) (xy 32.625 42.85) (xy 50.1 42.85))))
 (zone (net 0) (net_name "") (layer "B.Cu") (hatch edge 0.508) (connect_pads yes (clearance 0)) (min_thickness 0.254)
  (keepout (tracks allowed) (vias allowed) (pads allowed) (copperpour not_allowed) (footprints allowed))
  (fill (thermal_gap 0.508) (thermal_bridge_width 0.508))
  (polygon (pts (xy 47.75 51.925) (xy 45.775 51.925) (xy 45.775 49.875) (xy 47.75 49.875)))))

